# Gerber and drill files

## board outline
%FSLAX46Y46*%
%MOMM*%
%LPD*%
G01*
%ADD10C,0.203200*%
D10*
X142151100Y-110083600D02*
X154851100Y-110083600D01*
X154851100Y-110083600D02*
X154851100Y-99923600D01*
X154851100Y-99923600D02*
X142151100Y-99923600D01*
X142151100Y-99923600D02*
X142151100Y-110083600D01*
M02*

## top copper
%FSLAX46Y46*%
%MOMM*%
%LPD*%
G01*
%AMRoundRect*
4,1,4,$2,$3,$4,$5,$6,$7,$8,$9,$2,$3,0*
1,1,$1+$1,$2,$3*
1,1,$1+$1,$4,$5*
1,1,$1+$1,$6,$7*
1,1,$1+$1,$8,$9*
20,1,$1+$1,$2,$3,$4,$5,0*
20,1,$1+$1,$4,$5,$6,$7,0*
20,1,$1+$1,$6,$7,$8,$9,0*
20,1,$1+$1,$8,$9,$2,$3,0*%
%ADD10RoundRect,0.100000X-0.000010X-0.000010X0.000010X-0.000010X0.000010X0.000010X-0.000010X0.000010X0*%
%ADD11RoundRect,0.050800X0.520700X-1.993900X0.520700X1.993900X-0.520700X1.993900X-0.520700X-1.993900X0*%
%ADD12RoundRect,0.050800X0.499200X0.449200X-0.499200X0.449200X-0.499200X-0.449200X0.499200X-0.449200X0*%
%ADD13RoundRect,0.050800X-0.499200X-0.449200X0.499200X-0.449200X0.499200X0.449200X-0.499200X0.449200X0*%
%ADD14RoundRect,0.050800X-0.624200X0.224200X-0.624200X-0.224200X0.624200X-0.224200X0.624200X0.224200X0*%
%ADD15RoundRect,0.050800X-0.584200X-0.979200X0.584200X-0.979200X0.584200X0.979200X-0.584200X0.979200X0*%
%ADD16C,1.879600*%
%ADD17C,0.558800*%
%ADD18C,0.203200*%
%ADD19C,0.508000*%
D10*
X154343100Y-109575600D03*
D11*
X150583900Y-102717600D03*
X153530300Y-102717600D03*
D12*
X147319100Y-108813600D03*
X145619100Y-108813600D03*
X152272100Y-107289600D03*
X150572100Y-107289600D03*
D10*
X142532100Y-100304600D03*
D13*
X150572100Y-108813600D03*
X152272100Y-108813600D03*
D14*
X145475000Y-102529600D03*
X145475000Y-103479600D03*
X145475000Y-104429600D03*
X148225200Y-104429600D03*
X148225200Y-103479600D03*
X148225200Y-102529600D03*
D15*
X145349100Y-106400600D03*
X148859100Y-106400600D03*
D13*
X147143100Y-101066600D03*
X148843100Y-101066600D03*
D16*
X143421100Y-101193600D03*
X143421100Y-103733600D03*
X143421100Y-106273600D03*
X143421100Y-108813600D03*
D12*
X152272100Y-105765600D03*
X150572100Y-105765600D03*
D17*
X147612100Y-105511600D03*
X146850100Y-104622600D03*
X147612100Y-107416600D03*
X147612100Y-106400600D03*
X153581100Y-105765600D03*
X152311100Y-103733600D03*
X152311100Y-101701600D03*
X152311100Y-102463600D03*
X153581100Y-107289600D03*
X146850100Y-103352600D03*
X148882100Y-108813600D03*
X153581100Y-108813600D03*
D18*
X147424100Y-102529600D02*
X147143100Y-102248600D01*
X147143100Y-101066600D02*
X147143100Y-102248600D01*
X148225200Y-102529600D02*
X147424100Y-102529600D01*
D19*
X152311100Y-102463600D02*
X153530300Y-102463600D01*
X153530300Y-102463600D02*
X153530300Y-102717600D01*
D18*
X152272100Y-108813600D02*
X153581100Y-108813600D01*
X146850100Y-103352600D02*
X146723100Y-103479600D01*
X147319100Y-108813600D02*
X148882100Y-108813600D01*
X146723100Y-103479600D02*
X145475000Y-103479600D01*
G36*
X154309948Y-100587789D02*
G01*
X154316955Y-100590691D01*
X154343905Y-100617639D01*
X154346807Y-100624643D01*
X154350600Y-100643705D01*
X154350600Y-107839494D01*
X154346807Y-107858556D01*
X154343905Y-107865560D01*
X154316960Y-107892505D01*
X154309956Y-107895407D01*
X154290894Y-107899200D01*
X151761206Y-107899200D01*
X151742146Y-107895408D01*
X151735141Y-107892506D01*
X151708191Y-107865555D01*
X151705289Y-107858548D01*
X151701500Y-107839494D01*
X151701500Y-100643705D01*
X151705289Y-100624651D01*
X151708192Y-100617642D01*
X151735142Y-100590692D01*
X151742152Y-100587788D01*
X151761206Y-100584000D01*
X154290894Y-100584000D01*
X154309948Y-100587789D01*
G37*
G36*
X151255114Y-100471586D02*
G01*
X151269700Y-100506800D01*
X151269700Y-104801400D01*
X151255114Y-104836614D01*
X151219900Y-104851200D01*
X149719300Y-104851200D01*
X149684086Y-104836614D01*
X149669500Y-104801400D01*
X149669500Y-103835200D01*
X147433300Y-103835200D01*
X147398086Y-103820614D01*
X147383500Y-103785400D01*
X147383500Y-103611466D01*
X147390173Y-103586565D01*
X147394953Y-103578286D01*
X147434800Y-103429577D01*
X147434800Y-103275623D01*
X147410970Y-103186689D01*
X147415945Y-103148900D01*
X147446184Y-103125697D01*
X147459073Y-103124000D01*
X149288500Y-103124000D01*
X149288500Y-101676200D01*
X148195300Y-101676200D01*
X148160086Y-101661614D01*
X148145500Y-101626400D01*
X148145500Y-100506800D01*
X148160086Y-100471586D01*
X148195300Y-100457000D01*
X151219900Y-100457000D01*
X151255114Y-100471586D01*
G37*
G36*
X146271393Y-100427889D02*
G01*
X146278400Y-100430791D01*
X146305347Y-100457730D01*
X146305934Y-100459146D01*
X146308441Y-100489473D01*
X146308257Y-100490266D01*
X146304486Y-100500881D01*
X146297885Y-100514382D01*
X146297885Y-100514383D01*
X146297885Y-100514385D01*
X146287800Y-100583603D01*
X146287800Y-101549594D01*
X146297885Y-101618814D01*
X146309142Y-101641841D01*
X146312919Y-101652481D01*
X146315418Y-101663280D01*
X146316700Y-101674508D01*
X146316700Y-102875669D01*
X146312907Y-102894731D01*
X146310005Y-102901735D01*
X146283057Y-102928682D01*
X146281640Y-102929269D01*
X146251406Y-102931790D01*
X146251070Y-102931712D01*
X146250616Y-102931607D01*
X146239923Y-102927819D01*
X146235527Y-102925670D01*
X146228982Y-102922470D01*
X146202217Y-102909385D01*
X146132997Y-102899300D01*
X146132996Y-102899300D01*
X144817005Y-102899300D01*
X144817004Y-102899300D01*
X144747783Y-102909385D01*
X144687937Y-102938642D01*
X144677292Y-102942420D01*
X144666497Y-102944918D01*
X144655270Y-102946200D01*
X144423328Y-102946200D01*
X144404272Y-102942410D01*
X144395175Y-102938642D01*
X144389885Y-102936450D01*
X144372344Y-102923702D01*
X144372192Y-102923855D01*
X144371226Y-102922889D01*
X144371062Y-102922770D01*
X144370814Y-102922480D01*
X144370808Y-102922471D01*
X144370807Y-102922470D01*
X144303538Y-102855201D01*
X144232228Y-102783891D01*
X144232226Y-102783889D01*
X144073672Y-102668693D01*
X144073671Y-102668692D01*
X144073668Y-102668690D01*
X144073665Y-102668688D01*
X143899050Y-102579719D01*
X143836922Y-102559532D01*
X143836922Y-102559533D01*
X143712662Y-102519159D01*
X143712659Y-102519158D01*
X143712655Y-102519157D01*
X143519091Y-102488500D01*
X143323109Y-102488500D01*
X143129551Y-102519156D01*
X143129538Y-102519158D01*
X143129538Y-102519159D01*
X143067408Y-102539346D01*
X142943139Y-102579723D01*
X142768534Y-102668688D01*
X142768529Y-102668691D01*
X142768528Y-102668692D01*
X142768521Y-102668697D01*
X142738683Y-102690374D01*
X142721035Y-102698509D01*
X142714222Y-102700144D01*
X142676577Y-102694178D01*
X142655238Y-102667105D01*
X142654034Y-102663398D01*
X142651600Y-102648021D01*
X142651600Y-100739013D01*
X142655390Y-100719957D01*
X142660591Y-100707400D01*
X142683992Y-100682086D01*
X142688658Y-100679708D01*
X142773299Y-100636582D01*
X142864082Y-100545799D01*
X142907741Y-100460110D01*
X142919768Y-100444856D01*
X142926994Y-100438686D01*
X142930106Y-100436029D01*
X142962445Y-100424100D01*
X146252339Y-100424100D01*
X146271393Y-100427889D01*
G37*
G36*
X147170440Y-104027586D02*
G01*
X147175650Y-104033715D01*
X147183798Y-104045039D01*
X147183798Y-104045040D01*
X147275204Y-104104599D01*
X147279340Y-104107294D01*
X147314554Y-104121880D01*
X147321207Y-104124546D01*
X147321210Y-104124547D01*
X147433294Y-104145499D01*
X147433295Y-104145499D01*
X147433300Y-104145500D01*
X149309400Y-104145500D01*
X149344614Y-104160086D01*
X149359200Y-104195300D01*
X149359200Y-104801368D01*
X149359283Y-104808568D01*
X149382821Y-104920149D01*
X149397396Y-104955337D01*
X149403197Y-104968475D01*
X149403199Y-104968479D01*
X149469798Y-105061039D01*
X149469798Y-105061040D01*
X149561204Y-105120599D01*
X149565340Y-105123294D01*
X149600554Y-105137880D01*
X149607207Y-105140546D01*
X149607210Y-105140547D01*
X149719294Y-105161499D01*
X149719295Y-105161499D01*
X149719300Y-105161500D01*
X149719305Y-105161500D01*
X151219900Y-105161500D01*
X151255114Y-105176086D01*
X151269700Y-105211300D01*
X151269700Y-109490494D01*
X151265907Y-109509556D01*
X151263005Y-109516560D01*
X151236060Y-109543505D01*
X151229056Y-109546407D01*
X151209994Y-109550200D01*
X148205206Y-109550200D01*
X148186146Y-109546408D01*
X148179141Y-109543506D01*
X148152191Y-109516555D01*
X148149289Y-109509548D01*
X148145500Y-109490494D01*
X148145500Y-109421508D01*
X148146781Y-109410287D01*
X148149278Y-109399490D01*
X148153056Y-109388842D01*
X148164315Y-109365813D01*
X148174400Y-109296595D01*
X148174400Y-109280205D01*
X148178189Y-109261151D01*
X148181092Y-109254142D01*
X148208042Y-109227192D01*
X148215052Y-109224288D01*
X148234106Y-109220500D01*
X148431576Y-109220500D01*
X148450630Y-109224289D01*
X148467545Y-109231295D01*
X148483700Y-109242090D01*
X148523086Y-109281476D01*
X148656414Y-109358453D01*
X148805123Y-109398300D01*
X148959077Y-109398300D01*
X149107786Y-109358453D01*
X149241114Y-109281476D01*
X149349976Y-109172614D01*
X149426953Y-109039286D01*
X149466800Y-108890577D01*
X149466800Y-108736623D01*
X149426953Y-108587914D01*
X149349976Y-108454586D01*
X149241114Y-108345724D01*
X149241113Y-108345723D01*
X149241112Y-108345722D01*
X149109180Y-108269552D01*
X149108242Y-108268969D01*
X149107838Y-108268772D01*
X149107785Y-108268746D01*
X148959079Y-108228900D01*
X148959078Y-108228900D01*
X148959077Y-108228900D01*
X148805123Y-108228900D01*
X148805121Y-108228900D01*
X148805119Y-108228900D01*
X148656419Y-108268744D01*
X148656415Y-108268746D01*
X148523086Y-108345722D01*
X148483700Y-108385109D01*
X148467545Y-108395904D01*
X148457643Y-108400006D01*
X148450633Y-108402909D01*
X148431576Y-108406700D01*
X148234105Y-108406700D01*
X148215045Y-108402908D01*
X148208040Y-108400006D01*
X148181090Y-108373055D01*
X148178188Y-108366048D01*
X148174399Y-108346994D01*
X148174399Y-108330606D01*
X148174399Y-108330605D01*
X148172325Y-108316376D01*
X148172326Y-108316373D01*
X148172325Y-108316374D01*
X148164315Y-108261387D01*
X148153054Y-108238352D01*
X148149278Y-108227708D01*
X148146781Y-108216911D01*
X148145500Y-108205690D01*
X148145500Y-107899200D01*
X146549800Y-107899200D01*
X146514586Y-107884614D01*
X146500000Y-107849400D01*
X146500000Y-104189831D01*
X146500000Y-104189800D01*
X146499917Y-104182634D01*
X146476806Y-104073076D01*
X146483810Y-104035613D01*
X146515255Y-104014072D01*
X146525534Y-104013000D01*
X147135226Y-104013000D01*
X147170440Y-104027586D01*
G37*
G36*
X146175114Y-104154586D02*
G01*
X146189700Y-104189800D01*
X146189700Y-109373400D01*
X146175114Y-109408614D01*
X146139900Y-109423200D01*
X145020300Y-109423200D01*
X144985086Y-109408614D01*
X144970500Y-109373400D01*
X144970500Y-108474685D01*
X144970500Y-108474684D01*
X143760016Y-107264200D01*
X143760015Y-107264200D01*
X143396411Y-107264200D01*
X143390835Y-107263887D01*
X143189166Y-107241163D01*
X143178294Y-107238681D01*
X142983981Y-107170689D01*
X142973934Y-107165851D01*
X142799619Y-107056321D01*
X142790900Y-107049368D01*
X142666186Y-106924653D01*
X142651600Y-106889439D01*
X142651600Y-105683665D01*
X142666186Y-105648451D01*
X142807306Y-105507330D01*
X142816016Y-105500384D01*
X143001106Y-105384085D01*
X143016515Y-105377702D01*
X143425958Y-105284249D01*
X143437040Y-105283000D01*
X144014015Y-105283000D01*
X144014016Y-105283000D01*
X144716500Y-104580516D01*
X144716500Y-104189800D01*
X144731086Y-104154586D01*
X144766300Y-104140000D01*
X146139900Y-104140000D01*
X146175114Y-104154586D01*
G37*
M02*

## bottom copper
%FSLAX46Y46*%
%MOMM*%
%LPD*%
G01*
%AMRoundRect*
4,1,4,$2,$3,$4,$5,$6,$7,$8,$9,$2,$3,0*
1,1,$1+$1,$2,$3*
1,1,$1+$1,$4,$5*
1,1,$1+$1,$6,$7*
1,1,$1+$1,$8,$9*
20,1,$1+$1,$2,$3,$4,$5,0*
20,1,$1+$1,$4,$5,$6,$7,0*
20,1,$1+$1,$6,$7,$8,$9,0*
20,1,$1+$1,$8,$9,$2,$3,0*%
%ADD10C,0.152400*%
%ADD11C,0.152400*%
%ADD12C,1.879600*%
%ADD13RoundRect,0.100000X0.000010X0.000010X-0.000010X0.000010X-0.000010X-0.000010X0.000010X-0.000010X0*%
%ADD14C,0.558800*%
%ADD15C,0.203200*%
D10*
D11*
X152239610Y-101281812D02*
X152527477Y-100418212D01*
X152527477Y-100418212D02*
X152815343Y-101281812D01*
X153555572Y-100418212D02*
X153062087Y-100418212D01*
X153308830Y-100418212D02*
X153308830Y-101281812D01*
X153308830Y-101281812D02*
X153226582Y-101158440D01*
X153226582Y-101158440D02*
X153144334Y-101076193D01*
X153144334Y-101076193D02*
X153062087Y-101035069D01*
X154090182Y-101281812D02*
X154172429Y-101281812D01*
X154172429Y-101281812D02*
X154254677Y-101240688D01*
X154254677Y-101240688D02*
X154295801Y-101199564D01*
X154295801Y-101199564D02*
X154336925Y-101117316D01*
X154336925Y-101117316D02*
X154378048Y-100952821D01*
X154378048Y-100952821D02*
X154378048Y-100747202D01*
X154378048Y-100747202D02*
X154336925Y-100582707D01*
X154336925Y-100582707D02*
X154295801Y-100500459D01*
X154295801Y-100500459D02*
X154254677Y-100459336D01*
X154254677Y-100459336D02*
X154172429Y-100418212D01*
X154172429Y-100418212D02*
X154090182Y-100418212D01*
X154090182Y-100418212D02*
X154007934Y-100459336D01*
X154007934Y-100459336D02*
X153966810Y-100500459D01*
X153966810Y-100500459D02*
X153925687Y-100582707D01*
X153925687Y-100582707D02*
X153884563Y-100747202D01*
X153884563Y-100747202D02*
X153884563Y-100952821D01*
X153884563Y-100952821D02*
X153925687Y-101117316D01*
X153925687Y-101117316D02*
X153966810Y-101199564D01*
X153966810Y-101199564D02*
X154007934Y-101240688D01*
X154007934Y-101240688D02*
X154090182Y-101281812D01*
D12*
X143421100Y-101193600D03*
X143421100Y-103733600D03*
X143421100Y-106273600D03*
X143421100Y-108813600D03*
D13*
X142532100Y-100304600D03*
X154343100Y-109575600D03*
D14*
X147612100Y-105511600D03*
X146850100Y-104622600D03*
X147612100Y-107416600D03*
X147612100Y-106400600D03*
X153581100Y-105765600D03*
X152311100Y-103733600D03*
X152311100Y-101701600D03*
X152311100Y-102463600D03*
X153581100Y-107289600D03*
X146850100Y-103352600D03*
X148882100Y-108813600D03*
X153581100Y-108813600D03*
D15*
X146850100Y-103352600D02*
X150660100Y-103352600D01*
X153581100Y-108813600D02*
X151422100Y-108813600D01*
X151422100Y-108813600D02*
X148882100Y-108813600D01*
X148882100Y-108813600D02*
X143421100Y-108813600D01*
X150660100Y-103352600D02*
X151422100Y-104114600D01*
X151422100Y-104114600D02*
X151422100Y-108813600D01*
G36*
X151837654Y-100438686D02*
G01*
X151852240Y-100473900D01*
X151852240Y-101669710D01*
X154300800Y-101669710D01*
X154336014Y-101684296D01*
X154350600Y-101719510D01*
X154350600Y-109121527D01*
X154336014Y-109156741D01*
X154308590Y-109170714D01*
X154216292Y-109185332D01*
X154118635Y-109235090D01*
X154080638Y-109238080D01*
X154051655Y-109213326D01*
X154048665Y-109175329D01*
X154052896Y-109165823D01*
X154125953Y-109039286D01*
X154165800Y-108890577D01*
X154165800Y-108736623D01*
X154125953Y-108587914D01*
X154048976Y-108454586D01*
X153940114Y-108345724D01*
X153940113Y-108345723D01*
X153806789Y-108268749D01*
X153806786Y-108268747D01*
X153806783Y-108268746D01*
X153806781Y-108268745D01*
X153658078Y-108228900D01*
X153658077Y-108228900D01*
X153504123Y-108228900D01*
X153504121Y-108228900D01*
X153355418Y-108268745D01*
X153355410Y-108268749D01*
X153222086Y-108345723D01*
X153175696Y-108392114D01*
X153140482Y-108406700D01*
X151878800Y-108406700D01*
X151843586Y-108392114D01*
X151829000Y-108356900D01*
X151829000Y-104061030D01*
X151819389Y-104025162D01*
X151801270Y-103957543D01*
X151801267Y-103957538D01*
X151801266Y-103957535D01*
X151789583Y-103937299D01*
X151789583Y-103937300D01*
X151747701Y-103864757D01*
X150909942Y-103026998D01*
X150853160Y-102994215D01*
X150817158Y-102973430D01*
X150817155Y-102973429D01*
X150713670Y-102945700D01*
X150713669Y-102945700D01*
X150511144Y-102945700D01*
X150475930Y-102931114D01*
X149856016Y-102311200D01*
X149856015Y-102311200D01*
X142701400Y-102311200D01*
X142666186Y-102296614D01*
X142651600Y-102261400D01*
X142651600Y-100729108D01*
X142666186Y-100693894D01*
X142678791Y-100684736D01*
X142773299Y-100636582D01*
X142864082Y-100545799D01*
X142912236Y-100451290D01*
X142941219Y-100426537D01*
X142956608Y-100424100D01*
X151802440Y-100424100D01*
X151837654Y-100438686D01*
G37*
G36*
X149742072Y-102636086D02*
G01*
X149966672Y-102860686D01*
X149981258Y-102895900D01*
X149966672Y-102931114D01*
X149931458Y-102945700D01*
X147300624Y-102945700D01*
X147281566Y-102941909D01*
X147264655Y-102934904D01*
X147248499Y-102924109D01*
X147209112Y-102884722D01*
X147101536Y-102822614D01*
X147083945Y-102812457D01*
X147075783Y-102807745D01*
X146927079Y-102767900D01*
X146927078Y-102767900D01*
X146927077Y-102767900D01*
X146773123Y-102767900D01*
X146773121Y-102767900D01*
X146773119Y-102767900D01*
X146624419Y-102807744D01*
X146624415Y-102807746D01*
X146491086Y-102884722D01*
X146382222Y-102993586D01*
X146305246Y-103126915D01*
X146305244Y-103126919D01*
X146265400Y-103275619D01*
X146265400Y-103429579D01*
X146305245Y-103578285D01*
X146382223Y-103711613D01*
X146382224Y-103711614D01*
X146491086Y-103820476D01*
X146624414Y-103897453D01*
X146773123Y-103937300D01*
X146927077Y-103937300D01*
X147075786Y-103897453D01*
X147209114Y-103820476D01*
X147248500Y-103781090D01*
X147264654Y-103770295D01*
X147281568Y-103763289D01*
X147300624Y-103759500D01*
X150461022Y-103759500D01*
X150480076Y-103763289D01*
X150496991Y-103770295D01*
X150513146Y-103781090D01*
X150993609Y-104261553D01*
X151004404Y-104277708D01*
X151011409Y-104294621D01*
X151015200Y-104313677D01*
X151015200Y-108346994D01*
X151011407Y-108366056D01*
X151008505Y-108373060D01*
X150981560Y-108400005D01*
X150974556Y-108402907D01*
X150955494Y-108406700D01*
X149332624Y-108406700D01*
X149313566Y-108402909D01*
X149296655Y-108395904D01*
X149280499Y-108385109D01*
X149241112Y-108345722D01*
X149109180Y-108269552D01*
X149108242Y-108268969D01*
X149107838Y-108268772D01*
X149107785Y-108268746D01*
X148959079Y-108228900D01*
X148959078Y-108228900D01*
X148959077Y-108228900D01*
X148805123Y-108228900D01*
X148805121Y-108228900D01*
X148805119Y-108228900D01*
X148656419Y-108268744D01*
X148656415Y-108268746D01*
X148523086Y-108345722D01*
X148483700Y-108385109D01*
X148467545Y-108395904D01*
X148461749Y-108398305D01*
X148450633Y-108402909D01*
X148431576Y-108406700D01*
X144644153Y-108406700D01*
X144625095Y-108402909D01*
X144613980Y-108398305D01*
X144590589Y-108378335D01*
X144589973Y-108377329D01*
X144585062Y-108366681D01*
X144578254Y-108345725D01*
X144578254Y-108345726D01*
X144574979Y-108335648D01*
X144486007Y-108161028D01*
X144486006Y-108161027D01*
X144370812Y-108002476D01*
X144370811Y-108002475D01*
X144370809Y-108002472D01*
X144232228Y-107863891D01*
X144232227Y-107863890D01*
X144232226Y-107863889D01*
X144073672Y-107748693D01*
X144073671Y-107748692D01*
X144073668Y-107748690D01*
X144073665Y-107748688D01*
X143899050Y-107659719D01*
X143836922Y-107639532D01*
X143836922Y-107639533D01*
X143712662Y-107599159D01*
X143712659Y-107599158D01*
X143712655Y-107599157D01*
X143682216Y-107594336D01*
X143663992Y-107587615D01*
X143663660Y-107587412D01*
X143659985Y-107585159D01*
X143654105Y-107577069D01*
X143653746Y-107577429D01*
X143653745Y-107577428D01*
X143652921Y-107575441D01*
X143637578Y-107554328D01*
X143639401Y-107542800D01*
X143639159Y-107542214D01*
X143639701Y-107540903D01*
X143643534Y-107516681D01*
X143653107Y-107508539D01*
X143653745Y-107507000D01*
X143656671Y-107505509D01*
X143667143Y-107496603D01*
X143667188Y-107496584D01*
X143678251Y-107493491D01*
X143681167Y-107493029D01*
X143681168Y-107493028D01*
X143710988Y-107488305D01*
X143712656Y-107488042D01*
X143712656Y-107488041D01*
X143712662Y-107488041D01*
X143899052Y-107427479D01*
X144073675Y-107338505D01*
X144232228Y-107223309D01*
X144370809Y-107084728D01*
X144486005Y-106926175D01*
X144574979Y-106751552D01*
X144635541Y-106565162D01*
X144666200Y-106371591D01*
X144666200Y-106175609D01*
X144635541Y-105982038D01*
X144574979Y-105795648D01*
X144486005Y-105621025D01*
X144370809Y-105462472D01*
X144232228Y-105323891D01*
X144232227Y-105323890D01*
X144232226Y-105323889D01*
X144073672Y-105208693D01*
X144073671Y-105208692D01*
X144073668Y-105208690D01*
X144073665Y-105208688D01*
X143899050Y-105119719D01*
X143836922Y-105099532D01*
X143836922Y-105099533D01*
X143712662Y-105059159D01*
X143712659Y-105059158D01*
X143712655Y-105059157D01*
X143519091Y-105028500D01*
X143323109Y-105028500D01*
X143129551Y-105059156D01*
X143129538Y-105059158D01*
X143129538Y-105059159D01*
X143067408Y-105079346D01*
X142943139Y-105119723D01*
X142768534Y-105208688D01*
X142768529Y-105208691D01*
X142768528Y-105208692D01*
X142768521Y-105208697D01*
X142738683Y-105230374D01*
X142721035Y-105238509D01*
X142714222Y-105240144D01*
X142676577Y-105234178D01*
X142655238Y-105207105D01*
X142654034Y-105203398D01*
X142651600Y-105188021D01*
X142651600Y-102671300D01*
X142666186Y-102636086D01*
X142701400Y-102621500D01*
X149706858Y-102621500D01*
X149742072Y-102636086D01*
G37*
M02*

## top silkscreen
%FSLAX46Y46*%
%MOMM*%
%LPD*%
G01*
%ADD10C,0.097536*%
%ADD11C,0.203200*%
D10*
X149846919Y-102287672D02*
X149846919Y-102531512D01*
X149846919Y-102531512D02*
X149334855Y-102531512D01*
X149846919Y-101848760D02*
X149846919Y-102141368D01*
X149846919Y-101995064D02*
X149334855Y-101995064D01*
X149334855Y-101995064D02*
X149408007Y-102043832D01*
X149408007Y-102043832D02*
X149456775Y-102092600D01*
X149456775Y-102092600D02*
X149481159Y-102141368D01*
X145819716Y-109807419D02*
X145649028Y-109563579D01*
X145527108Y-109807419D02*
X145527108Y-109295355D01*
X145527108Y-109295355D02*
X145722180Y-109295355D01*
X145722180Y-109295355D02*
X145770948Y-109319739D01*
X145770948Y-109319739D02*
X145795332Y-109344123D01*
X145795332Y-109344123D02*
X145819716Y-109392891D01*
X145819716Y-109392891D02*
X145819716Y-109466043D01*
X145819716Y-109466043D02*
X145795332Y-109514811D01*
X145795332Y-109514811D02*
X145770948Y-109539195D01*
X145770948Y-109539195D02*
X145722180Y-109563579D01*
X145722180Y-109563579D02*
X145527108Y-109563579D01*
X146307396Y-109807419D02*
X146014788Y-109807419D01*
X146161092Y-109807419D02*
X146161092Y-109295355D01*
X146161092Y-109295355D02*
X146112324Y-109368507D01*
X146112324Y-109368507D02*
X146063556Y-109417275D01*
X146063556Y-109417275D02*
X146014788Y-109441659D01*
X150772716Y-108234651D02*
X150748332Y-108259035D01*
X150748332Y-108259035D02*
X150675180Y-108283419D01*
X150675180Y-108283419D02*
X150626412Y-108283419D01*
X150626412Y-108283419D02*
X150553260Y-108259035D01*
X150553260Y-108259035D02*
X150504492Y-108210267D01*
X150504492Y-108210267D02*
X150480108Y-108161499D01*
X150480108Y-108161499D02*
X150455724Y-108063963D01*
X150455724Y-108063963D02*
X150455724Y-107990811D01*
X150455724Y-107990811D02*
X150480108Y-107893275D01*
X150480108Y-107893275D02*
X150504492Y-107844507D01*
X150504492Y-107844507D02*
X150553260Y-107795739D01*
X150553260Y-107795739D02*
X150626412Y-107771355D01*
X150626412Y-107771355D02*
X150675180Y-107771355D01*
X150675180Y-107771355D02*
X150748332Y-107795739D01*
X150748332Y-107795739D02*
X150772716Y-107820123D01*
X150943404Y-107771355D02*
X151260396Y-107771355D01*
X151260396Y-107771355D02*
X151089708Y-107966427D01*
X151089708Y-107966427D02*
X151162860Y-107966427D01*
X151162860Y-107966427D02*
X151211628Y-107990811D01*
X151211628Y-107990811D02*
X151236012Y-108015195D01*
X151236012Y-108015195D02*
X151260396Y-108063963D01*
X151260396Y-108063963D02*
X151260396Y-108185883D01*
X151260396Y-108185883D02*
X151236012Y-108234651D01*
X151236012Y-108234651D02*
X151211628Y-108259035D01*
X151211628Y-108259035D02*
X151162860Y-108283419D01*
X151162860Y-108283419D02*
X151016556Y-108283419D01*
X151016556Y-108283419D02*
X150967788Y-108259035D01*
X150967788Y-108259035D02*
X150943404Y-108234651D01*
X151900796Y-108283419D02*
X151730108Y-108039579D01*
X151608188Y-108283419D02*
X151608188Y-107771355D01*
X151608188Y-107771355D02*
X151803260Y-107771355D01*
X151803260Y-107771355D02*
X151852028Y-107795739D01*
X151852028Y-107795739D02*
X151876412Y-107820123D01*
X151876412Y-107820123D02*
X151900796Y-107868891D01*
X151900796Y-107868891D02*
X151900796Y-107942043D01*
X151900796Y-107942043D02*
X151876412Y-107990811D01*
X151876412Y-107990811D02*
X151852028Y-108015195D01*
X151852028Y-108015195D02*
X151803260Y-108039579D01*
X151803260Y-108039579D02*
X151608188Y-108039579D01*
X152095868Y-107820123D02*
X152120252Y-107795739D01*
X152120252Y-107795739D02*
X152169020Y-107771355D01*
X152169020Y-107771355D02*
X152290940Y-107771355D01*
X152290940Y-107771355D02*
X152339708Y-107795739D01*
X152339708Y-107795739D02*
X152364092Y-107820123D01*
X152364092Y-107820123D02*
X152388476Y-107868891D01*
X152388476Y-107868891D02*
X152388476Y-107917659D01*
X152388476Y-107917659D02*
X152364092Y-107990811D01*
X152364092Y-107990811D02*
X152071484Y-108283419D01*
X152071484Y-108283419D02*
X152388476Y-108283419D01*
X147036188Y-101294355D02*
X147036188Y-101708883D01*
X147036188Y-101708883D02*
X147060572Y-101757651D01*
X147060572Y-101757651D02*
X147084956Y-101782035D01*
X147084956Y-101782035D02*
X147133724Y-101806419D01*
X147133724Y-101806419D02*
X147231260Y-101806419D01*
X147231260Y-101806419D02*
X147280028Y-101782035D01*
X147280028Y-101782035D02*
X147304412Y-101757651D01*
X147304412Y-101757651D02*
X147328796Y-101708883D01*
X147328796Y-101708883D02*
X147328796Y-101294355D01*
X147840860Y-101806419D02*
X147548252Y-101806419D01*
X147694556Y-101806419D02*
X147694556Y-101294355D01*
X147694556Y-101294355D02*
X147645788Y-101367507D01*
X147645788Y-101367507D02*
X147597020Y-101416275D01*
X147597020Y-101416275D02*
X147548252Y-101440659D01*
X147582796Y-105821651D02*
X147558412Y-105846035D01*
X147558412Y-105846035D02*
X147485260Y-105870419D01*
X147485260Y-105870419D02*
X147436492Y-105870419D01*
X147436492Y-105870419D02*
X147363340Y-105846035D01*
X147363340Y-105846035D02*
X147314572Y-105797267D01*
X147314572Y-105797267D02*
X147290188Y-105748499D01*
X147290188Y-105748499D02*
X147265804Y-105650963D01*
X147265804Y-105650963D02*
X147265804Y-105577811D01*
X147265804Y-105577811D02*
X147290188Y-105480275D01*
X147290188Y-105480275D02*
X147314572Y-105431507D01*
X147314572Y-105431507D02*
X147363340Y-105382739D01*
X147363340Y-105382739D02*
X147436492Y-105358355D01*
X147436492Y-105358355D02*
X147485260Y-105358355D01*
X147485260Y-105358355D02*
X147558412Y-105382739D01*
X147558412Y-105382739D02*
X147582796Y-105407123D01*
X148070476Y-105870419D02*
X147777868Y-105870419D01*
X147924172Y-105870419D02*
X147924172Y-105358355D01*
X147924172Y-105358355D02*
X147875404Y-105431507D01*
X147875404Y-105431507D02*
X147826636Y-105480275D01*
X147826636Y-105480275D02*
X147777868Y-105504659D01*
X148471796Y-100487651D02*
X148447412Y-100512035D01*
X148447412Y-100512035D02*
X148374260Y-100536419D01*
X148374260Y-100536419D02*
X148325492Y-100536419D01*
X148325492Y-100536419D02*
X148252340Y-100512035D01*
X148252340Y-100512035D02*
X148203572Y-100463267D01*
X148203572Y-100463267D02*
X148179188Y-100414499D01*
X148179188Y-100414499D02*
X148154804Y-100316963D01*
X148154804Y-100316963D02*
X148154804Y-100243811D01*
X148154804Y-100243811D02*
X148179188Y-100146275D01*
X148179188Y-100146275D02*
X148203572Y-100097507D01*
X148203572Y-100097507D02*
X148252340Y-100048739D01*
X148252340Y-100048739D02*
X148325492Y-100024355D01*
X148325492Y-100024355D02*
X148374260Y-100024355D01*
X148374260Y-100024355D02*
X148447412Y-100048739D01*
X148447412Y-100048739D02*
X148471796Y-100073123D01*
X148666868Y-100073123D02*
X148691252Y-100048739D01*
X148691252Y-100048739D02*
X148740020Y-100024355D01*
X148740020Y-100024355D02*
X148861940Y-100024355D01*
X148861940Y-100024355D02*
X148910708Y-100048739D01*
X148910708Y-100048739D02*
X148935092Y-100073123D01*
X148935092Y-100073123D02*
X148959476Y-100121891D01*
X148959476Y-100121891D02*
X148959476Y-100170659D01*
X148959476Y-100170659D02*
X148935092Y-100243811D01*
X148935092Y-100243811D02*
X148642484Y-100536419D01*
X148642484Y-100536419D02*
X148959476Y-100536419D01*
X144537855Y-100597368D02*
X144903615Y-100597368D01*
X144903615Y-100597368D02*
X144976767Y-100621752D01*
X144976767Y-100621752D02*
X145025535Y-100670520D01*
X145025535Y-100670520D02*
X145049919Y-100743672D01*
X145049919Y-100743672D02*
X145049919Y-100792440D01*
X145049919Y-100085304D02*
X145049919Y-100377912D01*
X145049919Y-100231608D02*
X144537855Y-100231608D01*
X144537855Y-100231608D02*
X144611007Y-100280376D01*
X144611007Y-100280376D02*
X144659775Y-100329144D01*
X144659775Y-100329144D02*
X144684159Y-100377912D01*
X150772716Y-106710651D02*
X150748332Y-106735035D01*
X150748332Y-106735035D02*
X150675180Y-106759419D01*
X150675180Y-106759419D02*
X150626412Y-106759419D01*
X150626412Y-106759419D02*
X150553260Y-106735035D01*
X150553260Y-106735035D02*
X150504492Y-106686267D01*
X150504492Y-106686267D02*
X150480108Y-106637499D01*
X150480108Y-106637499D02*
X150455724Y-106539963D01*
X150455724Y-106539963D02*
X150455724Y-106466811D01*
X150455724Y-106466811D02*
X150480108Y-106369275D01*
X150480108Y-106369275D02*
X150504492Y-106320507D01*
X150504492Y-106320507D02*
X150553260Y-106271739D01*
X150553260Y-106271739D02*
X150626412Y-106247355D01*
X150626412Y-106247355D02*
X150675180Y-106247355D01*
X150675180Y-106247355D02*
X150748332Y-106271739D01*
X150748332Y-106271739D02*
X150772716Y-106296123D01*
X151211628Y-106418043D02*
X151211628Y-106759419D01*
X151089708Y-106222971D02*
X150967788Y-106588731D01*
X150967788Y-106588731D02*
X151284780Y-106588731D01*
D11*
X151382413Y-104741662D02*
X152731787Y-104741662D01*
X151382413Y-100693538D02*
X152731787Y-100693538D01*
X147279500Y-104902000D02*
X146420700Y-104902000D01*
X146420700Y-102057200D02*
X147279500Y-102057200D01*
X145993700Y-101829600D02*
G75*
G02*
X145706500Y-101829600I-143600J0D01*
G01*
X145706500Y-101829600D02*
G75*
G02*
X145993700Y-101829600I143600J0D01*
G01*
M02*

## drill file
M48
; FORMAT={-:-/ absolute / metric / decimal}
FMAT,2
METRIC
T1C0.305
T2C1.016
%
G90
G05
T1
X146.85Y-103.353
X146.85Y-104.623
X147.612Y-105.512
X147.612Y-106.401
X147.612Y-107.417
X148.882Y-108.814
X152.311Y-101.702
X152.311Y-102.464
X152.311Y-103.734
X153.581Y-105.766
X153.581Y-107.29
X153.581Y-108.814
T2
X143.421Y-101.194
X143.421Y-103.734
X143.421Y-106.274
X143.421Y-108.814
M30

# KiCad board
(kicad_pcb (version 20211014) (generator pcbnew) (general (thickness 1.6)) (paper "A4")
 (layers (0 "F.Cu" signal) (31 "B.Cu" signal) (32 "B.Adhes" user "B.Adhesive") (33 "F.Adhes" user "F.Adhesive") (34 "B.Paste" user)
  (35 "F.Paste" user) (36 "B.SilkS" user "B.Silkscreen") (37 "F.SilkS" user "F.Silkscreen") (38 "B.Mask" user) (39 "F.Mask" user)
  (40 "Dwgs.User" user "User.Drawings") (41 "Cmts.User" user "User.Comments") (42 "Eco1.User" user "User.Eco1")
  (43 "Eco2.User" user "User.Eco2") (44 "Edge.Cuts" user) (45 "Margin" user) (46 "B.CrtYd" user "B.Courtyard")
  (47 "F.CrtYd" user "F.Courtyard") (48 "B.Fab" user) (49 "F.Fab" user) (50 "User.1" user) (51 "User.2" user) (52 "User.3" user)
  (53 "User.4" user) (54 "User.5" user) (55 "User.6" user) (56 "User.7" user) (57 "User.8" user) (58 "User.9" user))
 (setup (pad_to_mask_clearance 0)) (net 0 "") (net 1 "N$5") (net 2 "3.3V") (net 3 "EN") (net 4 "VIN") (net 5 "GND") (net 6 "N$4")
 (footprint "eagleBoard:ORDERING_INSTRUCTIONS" (layer "F.Cu") (at 166.2811 65.6336)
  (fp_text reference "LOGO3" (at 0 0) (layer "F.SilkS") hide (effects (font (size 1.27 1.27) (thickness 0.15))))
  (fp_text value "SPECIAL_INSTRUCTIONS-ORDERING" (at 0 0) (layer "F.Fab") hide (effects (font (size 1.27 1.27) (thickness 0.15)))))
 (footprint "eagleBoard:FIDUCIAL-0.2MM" (layer "F.Cu") (at 154.3431 109.5756)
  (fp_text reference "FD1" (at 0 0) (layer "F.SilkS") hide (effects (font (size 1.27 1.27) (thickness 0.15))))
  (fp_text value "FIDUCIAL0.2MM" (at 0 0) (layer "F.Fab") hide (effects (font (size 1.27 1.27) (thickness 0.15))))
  (pad "1" smd roundrect (at 0 0) (size 0.2 0.2) (layers "F.Cu") (roundrect_rratio 0.5) (solder_mask_margin 0.0635)))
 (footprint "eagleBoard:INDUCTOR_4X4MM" (layer "F.Cu") (at 152.0571 102.7176 90)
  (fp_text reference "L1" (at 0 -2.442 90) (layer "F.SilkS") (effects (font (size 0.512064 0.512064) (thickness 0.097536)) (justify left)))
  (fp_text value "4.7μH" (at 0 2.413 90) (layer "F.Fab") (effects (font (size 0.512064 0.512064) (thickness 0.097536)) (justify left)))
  (fp_line (start -2.024062 -0.674687) (end -2.024062 0.674687) (layer "F.SilkS") (width 0.2032))
  (fp_line (start 2.024062 -0.674687) (end 2.024062 0.674687) (layer "F.SilkS") (width 0.2032))
  (pad "P$1" smd roundrect (at 0 -1.4732 90) (size 4.0894 1.143) (layers "F.Cu" "F.Paste" "F.Mask") (roundrect_rratio 0.04444444444)
   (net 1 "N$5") (solder_mask_margin 0.0635))
  (pad "P$2" smd roundrect (at 0 1.4732 90) (size 4.0894 1.143) (layers "F.Cu" "F.Paste" "F.Mask") (roundrect_rratio 0.04444444444)
   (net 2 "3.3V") (solder_mask_margin 0.0635)))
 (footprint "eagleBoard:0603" (layer "F.Cu") (at 146.4691 108.8136 180)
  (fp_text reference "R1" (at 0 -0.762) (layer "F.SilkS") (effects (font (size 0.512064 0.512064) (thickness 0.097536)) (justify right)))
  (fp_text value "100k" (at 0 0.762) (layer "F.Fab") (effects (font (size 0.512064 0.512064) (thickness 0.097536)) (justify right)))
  (pad "1" smd roundrect (at -0.85 0 180) (size 1.1 1) (layers "F.Cu" "F.Paste" "F.Mask") (roundrect_rratio 0.0508) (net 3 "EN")
   (solder_mask_margin 0.0635))
  (pad "2" smd roundrect (at 0.85 0 180) (size 1.1 1) (layers "F.Cu" "F.Paste" "F.Mask") (roundrect_rratio 0.0508) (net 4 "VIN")
   (solder_mask_margin 0.0635)))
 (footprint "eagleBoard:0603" (layer "F.Cu") (at 151.4221 107.2896 180)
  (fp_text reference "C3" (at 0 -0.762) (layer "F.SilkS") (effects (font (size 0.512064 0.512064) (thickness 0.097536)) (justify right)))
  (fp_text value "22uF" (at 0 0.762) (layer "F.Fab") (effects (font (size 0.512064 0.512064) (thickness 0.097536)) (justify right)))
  (pad "1" smd roundrect (at -0.85 0 180) (size 1.1 1) (layers "F.Cu" "F.Paste" "F.Mask") (roundrect_rratio 0.0508) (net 2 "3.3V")
   (solder_mask_margin 0.0635))
  (pad "2" smd roundrect (at 0.85 0 180) (size 1.1 1) (layers "F.Cu" "F.Paste" "F.Mask") (roundrect_rratio 0.0508) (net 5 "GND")
   (solder_mask_margin 0.0635)))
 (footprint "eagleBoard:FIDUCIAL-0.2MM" (layer "F.Cu") (at 142.5321 100.3046)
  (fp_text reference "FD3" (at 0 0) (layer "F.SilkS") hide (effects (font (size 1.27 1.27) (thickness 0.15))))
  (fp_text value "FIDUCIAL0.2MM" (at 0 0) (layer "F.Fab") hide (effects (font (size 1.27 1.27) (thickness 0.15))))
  (pad "1" smd roundrect (at 0 0) (size 0.2 0.2) (layers "F.Cu") (roundrect_rratio 0.5) (solder_mask_margin 0.0635)))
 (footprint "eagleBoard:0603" (layer "F.Cu") (at 151.4221 108.8136)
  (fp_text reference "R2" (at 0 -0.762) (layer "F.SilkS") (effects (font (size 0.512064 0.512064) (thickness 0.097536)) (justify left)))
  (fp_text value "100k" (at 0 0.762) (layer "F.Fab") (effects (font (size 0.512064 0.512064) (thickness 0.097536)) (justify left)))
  (pad "1" smd roundrect (at -0.85 0) (size 1.1 1) (layers "F.Cu" "F.Paste" "F.Mask") (roundrect_rratio 0.0508) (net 5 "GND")
   (solder_mask_margin 0.0635))
  (pad "2" smd roundrect (at 0.85 0) (size 1.1 1) (layers "F.Cu" "F.Paste" "F.Mask") (roundrect_rratio 0.0508) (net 3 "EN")
   (solder_mask_margin 0.0635)))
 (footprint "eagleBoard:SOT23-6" (layer "F.Cu") (at 146.8501 103.4796 -90)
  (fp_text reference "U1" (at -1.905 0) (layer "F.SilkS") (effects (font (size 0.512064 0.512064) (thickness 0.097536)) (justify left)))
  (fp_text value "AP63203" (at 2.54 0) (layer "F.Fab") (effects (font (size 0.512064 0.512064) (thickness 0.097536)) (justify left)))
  (fp_line (start 1.4224 -0.4294) (end 1.4224 0.4294) (layer "F.SilkS") (width 0.2032))
  (fp_line (start -1.4224 0.4294) (end -1.4224 -0.4294) (layer "F.SilkS") (width 0.2032))
  (fp_circle (center -1.65 1) (end -1.5064 1) (layer "F.SilkS") (width 0.2032) (fill none))
  (pad "1" smd roundrect (at -0.95 1.3751 270) (size 0.55 1.35) (layers "F.Cu" "F.Paste" "F.Mask") (roundrect_rratio 0.09236363636)
   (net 2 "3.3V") (solder_mask_margin 0.0635))
  (pad "2" smd roundrect (at 0 1.3751 270) (size 0.55 1.35) (layers "F.Cu" "F.Paste" "F.Mask") (roundrect_rratio 0.09236363636) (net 3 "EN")
   (solder_mask_margin 0.0635))
  (pad "3" smd roundrect (at 0.95 1.3751 270) (size 0.55 1.35) (layers "F.Cu" "F.Paste" "F.Mask") (roundrect_rratio 0.09236363636)
   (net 4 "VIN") (solder_mask_margin 0.0635))
  (pad "4" smd roundrect (at 0.95 -1.3751 270) (size 0.55 1.35) (layers "F.Cu" "F.Paste" "F.Mask") (roundrect_rratio 0.09236363636)
   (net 5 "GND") (solder_mask_margin 0.0635))
  (pad "5" smd roundrect (at 0 -1.3751 270) (size 0.55 1.35) (layers "F.Cu" "F.Paste" "F.Mask") (roundrect_rratio 0.09236363636)
   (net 1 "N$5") (solder_mask_margin 0.0635))
  (pad "6" smd roundrect (at -0.95 -1.3751 270) (size 0.55 1.35) (layers "F.Cu" "F.Paste" "F.Mask") (roundrect_rratio 0.09236363636)
   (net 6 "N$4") (solder_mask_margin 0.0635)))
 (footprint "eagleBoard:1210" (layer "F.Cu") (at 147.1041 106.4006)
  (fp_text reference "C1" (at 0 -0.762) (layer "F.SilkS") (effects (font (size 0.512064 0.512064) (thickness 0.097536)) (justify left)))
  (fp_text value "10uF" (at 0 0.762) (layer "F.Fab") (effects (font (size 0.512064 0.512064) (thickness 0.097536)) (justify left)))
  (pad "1" smd roundrect (at -1.755 0) (size 1.27 2.06) (layers "F.Cu" "F.Paste" "F.Mask") (roundrect_rratio 0.04) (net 4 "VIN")
   (solder_mask_margin 0.0635))
  (pad "2" smd roundrect (at 1.755 0) (size 1.27 2.06) (layers "F.Cu" "F.Paste" "F.Mask") (roundrect_rratio 0.04) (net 5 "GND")
   (solder_mask_margin 0.0635)))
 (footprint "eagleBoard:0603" (layer "F.Cu") (at 147.9931 101.0666)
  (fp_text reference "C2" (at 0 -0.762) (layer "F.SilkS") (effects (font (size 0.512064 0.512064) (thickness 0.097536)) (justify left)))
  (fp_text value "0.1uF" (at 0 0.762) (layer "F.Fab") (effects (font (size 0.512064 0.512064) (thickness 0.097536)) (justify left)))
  (pad "1" smd roundrect (at -0.85 0) (size 1.1 1) (layers "F.Cu" "F.Paste" "F.Mask") (roundrect_rratio 0.0508) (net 6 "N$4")
   (solder_mask_margin 0.0635))
  (pad "2" smd roundrect (at 0.85 0) (size 1.1 1) (layers "F.Cu" "F.Paste" "F.Mask") (roundrect_rratio 0.0508) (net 1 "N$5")
   (solder_mask_margin 0.0635)))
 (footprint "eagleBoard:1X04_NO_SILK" (layer "F.Cu") (at 143.4211 101.1936 -90)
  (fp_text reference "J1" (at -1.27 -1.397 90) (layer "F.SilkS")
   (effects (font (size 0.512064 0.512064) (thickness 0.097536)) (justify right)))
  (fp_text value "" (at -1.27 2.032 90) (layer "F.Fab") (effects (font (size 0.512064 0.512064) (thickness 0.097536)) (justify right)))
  (pad "1" thru_hole circle (at 0 0) (size 1.8796 1.8796) (drill 1.016) (layers *.Cu *.Mask) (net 2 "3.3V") (solder_mask_margin 0.0635))
  (pad "2" thru_hole circle (at 2.54 0) (size 1.8796 1.8796) (drill 1.016) (layers *.Cu *.Mask) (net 5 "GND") (solder_mask_margin 0.0635))
  (pad "3" thru_hole circle (at 5.08 0) (size 1.8796 1.8796) (drill 1.016) (layers *.Cu *.Mask) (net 4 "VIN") (solder_mask_margin 0.0635))
  (pad "4" thru_hole circle (at 7.62 0) (size 1.8796 1.8796) (drill 1.016) (layers *.Cu *.Mask) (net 3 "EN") (solder_mask_margin 0.0635)))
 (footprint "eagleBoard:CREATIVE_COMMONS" (layer "F.Cu") (at 125.6411 125.3236)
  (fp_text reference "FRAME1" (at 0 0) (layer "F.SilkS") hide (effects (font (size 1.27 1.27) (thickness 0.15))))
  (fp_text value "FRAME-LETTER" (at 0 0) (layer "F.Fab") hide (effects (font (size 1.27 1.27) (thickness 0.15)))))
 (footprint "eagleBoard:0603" (layer "F.Cu") (at 151.4221 105.7656 180)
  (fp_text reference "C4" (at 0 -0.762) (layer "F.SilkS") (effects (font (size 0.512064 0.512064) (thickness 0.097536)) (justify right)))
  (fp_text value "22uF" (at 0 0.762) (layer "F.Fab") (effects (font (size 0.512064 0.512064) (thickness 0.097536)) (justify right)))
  (pad "1" smd roundrect (at -0.85 0 180) (size 1.1 1) (layers "F.Cu" "F.Paste" "F.Mask") (roundrect_rratio 0.0508) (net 2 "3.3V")
   (solder_mask_margin 0.0635))
  (pad "2" smd roundrect (at 0.85 0 180) (size 1.1 1) (layers "F.Cu" "F.Paste" "F.Mask") (roundrect_rratio 0.0508) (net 5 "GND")
   (solder_mask_margin 0.0635)))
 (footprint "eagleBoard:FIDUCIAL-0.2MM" (layer "B.Cu") (at 142.5321 100.3046 180)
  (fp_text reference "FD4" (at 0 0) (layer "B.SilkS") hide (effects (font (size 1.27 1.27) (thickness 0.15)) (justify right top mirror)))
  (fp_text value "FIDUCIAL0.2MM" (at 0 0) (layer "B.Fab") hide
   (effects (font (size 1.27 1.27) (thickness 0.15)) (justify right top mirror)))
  (pad "1" smd roundrect (at 0 0 180) (size 0.2 0.2) (layers "B.Cu") (roundrect_rratio 0.5) (solder_mask_margin 0.0635)))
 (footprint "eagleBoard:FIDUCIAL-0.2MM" (layer "B.Cu") (at 154.3431 109.5756 180)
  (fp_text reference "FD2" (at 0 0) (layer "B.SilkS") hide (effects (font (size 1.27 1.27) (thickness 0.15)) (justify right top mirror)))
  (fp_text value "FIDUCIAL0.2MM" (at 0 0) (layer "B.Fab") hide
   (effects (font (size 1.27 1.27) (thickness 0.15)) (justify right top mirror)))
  (pad "1" smd roundrect (at 0 0 180) (size 0.2 0.2) (layers "B.Cu") (roundrect_rratio 0.5) (solder_mask_margin 0.0635)))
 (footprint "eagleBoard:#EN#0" (layer "B.Cu") (at 145.5801 108.8136 180)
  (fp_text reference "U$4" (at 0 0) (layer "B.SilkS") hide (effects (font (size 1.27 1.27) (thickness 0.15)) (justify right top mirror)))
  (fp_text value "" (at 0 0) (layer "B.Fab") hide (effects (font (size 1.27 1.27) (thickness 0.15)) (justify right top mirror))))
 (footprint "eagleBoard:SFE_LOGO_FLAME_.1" (layer "B.Cu") (at 149.8981 107.0356 180)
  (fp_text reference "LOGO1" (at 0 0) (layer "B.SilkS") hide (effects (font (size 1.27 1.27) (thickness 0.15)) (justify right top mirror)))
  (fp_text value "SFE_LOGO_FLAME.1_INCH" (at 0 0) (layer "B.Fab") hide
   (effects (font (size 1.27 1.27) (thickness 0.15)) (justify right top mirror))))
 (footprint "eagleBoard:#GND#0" (layer "B.Cu") (at 145.9611 103.7336 180)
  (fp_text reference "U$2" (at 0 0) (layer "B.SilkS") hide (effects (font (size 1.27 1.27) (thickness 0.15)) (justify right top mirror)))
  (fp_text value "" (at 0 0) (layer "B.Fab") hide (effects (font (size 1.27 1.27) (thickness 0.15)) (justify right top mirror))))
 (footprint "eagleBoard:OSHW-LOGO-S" (layer "B.Cu") (at 152.8191 107.0356 180)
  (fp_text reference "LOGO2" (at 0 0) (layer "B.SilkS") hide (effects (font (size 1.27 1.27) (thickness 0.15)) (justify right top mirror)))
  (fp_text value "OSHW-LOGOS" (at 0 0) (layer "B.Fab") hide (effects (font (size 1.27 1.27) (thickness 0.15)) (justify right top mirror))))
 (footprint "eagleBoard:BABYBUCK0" (layer "B.Cu") (at 154.8511 102.9716 180)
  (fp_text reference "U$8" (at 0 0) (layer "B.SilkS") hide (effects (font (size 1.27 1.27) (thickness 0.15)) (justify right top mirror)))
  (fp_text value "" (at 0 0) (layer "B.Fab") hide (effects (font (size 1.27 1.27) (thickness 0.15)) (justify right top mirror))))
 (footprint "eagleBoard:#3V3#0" (layer "B.Cu") (at 145.9611 101.1936 180)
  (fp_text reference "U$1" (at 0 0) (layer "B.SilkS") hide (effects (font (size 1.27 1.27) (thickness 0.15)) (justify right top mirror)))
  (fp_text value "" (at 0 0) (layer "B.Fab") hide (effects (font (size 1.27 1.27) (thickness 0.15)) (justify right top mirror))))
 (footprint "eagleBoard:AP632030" (layer "B.Cu") (at 151.2951 104.3686 180)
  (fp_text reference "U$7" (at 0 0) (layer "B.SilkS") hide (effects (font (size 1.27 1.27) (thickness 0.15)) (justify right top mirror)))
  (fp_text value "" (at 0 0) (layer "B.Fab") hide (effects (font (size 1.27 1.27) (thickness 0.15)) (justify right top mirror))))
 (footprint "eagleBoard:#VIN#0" (layer "B.Cu") (at 145.7071 106.2736 180)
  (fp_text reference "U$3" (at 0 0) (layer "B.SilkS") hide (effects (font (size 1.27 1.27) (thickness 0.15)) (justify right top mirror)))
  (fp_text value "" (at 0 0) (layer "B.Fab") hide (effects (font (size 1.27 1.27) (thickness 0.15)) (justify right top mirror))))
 (gr_line (start 142.1511 110.0836) (end 154.8511 110.0836) (layer "Edge.Cuts") (width 0.2032))
 (gr_line (start 154.8511 110.0836) (end 154.8511 99.9236) (layer "Edge.Cuts") (width 0.2032))
 (gr_line (start 154.8511 99.9236) (end 142.1511 99.9236) (layer "Edge.Cuts") (width 0.2032))
 (gr_line (start 142.1511 99.9236) (end 142.1511 110.0836) (layer "Edge.Cuts") (width 0.2032))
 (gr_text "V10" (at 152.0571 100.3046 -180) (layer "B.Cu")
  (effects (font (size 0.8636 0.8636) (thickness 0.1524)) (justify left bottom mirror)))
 (via (at 147.6121 105.5116) (size 0.5588) (drill 0.3048) (layers "F.Cu" "B.Cu") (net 5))
 (via (at 146.8501 104.6226) (size 0.5588) (drill 0.3048) (layers "F.Cu" "B.Cu") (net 5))
 (via (at 147.6121 107.4166) (size 0.5588) (drill 0.3048) (layers "F.Cu" "B.Cu") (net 5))
 (via (at 147.6121 106.4006) (size 0.5588) (drill 0.3048) (layers "F.Cu" "B.Cu") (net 5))
 (segment (start 147.4241 102.5296) (end 147.1431 102.2486) (width 0.2032) (layer "F.Cu") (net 6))
 (segment (start 147.1431 101.0666) (end 147.1431 102.2486) (width 0.2032) (layer "F.Cu") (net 6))
 (segment (start 148.2252 102.5296) (end 147.4241 102.5296) (width 0.2032) (layer "F.Cu") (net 6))
 (segment (start 152.3111 102.4636) (end 153.5303 102.4636) (width 0.508) (layer "F.Cu") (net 2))
 (segment (start 153.5303 102.4636) (end 153.5303 102.7176) (width 0.508) (layer "F.Cu") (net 2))
 (via (at 153.5811 105.7656) (size 0.5588) (drill 0.3048) (layers "F.Cu" "B.Cu") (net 2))
 (via (at 152.3111 103.7336) (size 0.5588) (drill 0.3048) (layers "F.Cu" "B.Cu") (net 2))
 (via (at 152.3111 101.7016) (size 0.5588) (drill 0.3048) (layers "F.Cu" "B.Cu") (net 2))
 (via (at 152.3111 102.4636) (size 0.5588) (drill 0.3048) (layers "F.Cu" "B.Cu") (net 2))
 (via (at 153.5811 107.2896) (size 0.5588) (drill 0.3048) (layers "F.Cu" "B.Cu") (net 2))
 (segment (start 152.2721 108.8136) (end 153.5811 108.8136) (width 0.2032) (layer "F.Cu") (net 3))
 (segment (start 146.8501 103.3526) (end 146.7231 103.4796) (width 0.2032) (layer "F.Cu") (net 3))
 (segment (start 147.3191 108.8136) (end 148.8821 108.8136) (width 0.2032) (layer "F.Cu") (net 3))
 (segment (start 146.7231 103.4796) (end 145.475 103.4796) (width 0.2032) (layer "F.Cu") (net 3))
 (via (at 146.8501 103.3526) (size 0.5588) (drill 0.3048) (layers "F.Cu" "B.Cu") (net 3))
 (via (at 148.8821 108.8136) (size 0.5588) (drill 0.3048) (layers "F.Cu" "B.Cu") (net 3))
 (via (at 153.5811 108.8136) (size 0.5588) (drill 0.3048) (layers "F.Cu" "B.Cu") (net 3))
 (segment (start 146.8501 103.3526) (end 150.6601 103.3526) (width 0.2032) (layer "B.Cu") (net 3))
 (segment (start 153.5811 108.8136) (end 151.4221 108.8136) (width 0.2032) (layer "B.Cu") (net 3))
 (segment (start 151.4221 108.8136) (end 148.8821 108.8136) (width 0.2032) (layer "B.Cu") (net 3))
 (segment (start 148.8821 108.8136) (end 143.4211 108.8136) (width 0.2032) (layer "B.Cu") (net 3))
 (segment (start 150.6601 103.3526) (end 151.4221 104.1146) (width 0.2032) (layer "B.Cu") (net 3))
 (segment (start 151.4221 104.1146) (end 151.4221 108.8136) (width 0.2032) (layer "B.Cu") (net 3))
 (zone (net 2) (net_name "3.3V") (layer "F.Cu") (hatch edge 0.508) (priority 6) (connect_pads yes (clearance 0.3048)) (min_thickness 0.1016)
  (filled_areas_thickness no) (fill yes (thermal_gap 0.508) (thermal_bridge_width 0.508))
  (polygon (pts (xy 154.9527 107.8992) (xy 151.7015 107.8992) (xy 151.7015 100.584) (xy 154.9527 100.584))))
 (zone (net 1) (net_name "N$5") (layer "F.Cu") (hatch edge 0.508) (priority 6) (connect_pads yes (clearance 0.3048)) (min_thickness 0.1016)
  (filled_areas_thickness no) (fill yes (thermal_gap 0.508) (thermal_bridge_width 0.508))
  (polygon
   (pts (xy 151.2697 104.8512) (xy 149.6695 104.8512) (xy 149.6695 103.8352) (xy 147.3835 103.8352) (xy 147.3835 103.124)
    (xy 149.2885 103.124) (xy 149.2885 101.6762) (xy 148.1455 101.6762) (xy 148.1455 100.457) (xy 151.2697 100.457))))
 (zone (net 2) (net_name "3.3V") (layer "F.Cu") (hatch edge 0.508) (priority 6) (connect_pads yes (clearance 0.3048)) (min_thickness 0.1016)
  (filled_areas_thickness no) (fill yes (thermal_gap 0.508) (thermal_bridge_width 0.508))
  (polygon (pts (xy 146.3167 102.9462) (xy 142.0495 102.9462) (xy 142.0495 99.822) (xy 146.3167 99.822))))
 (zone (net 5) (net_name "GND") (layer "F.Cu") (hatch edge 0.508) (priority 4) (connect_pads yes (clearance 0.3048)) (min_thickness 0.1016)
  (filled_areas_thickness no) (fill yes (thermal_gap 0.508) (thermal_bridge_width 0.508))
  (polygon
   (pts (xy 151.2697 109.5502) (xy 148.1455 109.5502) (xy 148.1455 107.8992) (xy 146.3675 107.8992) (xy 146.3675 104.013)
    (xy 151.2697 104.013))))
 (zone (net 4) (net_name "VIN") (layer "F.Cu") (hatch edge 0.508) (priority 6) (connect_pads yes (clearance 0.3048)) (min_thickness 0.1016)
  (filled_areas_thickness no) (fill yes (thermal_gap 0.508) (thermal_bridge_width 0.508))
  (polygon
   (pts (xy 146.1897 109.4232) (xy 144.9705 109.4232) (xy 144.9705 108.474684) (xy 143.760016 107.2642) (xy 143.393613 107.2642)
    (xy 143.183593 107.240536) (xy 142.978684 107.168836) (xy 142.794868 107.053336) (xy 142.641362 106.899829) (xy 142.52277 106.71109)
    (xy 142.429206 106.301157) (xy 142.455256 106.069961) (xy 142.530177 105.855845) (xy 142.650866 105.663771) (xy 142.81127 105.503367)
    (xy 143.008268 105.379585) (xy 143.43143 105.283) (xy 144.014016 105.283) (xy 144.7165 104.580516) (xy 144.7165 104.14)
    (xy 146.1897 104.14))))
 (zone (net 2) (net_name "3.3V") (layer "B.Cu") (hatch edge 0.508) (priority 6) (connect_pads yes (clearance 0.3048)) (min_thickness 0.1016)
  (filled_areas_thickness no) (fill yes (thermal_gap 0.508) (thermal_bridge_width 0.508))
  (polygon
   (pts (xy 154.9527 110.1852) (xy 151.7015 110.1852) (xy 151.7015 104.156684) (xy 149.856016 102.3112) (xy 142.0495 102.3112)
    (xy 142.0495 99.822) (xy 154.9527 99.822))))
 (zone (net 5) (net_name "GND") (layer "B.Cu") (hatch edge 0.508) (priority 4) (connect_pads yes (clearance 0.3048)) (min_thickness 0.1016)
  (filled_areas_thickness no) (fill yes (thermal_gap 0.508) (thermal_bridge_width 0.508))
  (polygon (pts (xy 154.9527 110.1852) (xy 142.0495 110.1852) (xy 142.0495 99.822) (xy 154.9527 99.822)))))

